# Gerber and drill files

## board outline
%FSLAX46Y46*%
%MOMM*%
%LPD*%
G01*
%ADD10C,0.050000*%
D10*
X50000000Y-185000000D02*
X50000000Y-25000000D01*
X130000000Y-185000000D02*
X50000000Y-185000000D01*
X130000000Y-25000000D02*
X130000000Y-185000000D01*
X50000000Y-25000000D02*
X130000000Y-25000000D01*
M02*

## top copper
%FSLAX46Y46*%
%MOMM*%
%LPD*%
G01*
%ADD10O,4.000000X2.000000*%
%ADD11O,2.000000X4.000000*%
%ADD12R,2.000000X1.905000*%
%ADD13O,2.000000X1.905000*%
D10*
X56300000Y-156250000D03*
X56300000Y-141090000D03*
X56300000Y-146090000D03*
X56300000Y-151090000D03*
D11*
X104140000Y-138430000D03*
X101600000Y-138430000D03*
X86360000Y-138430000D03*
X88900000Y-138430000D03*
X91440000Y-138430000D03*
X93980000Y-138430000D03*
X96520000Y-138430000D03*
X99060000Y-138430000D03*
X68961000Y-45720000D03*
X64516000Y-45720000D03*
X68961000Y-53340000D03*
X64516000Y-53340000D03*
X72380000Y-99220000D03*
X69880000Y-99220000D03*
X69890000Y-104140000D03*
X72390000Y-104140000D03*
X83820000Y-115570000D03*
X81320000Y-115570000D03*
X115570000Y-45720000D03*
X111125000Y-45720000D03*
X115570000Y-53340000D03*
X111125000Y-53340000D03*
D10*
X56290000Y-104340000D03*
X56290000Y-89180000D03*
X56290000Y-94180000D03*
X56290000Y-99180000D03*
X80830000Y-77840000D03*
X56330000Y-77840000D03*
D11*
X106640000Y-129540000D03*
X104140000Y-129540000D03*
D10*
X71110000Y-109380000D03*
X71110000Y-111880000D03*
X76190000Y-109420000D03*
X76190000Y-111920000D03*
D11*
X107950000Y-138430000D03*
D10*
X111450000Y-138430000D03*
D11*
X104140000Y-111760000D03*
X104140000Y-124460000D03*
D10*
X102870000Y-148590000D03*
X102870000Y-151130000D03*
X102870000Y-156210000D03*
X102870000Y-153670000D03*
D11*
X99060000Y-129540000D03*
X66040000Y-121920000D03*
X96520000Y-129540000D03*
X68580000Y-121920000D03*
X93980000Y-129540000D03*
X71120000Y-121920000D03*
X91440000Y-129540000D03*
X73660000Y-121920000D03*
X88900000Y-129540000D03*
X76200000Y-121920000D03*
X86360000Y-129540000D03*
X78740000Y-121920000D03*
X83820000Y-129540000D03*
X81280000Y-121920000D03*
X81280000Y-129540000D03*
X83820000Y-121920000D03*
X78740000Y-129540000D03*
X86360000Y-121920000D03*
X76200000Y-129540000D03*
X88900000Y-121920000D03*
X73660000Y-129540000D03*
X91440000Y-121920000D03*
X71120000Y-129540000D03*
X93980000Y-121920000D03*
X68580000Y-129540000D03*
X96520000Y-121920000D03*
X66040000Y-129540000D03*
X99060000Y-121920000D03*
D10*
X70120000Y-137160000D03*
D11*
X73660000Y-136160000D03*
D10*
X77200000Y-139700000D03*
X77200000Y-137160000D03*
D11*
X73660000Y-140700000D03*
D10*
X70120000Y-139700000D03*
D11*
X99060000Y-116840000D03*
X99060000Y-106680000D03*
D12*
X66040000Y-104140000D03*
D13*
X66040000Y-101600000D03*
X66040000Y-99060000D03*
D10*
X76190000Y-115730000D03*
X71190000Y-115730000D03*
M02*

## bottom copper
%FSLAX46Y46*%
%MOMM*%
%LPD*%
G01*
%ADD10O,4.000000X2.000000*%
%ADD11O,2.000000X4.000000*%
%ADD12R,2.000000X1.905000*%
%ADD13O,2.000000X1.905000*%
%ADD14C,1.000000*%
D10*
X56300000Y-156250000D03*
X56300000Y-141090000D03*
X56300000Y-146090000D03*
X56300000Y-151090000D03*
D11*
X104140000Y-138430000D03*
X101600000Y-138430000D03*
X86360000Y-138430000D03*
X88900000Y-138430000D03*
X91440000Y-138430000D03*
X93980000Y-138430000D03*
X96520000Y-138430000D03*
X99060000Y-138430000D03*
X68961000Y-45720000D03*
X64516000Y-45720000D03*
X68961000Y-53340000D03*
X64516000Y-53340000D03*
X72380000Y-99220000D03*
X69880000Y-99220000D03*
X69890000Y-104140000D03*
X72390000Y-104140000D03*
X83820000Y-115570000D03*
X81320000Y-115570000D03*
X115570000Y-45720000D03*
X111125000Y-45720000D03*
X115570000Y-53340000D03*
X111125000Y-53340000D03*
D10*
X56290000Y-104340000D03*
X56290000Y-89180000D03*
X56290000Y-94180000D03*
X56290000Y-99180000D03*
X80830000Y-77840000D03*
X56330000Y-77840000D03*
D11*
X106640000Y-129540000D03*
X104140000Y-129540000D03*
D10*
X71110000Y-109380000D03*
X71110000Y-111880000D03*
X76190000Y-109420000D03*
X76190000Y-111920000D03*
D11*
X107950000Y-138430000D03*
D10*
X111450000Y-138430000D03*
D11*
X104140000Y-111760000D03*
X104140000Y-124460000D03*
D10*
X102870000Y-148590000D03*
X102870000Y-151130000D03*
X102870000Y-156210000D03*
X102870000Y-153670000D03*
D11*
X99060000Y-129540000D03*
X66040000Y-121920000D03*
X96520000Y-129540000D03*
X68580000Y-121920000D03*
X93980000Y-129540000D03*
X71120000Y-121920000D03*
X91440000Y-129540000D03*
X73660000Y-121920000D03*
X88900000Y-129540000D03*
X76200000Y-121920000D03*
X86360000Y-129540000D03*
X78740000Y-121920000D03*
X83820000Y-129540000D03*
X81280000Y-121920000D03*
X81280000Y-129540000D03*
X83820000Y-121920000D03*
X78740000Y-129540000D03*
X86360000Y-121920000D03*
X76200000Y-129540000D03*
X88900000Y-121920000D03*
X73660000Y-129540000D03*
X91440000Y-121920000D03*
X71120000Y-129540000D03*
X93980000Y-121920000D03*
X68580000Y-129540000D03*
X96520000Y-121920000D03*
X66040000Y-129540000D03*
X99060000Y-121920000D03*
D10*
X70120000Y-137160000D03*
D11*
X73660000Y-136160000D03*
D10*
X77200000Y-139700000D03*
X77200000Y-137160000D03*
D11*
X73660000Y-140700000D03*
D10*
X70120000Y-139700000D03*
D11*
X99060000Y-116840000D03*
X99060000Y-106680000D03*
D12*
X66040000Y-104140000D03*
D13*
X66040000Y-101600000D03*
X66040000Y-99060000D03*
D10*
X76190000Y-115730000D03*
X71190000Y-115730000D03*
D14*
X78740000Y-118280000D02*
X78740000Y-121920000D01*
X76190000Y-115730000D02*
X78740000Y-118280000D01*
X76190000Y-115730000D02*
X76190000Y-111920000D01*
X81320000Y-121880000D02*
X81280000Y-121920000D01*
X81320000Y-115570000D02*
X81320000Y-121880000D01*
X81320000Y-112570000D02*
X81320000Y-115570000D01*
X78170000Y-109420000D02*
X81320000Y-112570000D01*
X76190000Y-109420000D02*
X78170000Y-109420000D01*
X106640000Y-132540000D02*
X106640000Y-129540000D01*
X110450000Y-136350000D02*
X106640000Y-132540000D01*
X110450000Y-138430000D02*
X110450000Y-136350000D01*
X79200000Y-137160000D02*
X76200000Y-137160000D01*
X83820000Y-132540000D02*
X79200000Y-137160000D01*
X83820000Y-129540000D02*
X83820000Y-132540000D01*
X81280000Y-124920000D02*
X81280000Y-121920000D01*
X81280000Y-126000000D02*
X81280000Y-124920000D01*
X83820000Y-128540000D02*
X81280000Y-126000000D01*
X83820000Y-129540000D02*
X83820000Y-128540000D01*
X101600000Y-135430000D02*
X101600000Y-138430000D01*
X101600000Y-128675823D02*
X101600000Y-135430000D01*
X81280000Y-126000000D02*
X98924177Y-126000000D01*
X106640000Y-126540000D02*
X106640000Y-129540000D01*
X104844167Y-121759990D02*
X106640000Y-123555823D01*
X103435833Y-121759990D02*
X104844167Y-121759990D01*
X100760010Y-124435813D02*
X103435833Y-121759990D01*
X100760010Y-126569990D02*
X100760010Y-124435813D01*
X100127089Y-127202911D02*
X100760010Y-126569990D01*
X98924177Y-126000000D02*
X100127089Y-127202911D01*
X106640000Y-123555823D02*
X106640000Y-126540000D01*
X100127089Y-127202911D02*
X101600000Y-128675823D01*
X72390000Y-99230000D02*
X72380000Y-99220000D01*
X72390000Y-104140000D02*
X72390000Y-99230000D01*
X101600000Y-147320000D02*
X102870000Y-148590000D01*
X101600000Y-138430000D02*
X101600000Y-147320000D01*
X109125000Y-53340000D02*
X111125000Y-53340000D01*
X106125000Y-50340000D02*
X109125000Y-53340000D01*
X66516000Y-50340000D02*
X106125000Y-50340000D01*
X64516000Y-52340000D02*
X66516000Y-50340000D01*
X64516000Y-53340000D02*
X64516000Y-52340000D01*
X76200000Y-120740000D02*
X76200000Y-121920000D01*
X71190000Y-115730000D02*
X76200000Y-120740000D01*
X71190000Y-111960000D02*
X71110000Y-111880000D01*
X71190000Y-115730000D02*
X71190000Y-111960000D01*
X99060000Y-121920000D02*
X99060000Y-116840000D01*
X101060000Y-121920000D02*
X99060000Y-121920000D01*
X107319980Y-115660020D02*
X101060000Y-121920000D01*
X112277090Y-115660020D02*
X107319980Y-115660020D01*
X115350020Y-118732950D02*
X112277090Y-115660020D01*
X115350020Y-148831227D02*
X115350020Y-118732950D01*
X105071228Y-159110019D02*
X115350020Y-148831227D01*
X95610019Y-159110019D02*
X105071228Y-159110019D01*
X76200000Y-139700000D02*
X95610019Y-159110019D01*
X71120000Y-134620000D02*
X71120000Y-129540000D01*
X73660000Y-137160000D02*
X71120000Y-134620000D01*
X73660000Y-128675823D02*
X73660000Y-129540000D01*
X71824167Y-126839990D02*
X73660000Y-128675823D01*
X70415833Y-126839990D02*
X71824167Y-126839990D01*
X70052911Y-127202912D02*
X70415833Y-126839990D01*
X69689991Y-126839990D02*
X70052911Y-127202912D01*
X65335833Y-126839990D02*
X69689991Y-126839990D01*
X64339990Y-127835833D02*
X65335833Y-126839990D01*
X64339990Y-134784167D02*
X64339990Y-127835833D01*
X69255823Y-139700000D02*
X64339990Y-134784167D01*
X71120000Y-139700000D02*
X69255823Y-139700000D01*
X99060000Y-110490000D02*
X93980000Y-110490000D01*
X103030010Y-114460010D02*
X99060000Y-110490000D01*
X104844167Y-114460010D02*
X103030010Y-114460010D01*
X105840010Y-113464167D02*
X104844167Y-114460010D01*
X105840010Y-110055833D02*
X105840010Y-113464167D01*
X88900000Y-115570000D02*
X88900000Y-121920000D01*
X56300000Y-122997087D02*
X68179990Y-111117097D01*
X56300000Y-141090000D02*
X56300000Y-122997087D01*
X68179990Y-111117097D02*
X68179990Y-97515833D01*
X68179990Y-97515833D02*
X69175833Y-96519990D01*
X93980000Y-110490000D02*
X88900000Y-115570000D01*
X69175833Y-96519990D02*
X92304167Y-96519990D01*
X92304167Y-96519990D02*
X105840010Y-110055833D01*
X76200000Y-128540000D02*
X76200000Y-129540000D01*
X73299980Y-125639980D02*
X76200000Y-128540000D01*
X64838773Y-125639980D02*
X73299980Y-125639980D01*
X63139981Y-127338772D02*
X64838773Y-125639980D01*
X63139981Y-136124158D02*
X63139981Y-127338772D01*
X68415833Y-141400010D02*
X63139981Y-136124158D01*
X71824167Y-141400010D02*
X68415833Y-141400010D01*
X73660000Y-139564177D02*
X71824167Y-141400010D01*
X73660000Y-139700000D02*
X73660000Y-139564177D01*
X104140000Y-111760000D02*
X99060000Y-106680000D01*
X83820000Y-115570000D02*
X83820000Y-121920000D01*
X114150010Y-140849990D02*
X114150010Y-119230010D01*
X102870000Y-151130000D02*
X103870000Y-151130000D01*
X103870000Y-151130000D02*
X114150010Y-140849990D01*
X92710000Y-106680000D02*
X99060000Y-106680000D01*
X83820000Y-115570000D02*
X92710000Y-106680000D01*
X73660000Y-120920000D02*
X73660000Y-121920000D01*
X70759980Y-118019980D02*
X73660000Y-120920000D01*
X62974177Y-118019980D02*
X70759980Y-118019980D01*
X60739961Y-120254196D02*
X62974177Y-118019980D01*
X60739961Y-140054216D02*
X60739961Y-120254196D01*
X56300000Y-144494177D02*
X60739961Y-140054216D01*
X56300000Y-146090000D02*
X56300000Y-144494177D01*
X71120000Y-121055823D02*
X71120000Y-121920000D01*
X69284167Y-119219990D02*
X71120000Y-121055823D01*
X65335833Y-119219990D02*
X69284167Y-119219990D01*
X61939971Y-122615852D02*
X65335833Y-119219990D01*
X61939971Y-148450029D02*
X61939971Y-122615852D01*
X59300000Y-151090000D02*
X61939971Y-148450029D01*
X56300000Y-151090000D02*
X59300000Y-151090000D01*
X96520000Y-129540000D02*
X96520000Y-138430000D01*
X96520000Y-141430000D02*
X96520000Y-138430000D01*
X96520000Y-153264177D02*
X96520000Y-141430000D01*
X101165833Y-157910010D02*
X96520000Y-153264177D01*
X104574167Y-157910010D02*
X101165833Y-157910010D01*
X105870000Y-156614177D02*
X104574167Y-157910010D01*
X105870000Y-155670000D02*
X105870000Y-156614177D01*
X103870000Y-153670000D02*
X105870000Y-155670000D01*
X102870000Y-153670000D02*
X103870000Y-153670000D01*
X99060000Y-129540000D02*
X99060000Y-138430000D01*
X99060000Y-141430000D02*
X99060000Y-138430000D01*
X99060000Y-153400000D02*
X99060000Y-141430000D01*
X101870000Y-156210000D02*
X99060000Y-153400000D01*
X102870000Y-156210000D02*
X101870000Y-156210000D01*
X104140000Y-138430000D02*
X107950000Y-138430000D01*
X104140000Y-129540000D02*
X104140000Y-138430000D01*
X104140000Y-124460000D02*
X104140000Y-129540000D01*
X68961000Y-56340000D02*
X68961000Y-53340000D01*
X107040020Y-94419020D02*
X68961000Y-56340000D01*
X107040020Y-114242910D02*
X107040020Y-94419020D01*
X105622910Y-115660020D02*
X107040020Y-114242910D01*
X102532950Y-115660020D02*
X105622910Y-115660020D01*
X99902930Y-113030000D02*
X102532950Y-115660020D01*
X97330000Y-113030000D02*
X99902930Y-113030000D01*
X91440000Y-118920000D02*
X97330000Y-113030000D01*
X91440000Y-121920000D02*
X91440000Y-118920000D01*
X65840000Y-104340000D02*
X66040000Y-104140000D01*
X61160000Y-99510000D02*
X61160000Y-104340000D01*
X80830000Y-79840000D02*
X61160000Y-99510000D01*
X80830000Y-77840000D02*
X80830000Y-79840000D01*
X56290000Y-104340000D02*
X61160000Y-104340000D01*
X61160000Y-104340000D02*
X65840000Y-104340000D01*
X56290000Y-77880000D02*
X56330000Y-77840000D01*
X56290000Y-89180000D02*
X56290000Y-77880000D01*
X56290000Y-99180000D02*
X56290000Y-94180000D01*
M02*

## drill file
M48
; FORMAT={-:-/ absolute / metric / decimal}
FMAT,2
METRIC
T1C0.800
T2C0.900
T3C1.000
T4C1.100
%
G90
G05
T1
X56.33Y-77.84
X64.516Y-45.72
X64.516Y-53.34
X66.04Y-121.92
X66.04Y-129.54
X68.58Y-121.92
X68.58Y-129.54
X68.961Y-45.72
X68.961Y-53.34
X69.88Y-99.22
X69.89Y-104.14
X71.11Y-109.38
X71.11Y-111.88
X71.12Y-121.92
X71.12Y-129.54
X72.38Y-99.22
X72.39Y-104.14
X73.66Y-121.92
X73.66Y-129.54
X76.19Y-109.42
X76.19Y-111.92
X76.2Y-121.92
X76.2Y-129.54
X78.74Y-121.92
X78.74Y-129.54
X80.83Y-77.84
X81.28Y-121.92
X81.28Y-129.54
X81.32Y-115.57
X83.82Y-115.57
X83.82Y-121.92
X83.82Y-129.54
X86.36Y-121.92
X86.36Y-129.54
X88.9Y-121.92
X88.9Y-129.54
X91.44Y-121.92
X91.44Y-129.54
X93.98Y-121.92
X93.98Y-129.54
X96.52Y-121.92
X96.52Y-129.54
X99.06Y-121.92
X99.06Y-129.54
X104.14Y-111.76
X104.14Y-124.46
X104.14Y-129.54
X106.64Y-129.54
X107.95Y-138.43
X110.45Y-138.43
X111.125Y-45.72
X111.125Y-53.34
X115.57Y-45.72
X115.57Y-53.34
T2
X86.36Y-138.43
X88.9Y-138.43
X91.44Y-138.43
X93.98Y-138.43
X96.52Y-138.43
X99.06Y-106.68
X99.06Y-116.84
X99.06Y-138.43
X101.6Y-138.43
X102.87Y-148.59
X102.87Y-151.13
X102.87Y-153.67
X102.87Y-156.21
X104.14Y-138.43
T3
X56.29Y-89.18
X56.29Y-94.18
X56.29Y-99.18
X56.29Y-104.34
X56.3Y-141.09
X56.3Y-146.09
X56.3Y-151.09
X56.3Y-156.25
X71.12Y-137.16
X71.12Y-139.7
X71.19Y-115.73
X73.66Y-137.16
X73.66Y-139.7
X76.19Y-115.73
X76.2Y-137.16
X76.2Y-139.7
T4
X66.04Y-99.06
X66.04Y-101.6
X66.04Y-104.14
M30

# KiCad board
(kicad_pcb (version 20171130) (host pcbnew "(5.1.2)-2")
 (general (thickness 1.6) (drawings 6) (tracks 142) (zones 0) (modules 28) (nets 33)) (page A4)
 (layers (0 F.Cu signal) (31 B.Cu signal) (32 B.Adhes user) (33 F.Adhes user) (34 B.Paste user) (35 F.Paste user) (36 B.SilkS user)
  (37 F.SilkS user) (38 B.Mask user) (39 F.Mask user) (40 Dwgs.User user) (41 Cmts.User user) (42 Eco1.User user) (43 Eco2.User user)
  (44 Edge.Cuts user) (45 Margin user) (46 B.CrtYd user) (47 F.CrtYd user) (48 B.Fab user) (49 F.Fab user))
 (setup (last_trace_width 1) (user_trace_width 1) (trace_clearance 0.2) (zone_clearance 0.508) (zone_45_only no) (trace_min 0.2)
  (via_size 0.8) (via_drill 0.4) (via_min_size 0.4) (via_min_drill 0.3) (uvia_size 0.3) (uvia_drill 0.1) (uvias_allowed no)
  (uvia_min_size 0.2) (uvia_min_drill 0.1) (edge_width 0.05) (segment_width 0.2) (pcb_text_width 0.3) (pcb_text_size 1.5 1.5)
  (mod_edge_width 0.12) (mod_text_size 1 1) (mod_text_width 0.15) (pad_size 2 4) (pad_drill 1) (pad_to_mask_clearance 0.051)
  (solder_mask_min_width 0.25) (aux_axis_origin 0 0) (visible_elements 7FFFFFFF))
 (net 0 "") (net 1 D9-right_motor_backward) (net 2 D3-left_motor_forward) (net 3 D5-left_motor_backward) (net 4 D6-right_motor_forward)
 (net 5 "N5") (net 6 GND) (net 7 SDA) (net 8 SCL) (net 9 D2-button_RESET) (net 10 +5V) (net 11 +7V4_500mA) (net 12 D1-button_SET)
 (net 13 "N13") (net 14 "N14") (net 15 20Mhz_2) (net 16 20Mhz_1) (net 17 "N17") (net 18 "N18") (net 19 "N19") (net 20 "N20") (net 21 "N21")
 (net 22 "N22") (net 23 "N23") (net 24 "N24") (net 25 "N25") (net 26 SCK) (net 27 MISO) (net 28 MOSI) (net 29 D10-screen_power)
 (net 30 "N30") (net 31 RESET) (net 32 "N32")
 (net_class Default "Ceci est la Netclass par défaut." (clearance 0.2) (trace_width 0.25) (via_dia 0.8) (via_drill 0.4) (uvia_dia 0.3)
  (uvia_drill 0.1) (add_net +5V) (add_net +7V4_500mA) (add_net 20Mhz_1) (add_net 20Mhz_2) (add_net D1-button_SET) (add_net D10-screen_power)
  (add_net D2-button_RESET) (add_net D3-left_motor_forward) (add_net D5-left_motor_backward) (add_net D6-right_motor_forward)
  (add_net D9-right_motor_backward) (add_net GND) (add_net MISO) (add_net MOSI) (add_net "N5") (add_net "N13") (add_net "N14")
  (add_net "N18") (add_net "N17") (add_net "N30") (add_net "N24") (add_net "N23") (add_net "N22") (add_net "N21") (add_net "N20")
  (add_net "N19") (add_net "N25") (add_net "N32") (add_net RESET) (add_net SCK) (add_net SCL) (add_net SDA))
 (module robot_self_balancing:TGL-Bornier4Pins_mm (layer F.Cu) (at 50.8 148.59 90)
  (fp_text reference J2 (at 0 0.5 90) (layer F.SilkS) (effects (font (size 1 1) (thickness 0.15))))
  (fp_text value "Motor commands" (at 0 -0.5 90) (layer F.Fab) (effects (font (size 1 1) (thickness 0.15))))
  (pad 5 thru_hole oval (at -7.66 5.5 90) (size 2 4) (drill 1) (layers *.Cu *.Mask) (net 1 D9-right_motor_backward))
  (pad 8 thru_hole oval (at 7.5 5.5 270) (size 2 4) (drill 1) (layers *.Cu *.Mask) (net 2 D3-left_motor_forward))
  (pad 7 thru_hole oval (at 2.5 5.5 90) (size 2 4) (drill 1) (layers *.Cu *.Mask) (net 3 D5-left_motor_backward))
  (pad 6 thru_hole oval (at -2.5 5.5 90) (size 2 4) (drill 1) (layers *.Cu *.Mask) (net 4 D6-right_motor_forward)))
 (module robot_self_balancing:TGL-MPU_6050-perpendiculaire (layer F.Cu) (at 95.25 142.24 180)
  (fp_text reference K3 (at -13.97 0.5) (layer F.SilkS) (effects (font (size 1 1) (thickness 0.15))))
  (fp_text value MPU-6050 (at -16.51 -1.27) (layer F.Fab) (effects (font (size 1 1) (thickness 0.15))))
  (pad 13 thru_hole oval (at -8.89 3.81 180) (size 2 4) (drill 0.9) (layers *.Cu *.Mask) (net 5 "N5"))
  (pad 18 thru_hole oval (at -6.35 3.81 180) (size 2 4) (drill 0.9) (layers *.Cu *.Mask) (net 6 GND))
  (pad "" thru_hole oval (at 8.89 3.81 180) (size 2 4) (drill 0.9) (layers *.Cu *.Mask))
  (pad "" thru_hole oval (at 6.35 3.81 180) (size 2 4) (drill 0.9) (layers *.Cu *.Mask))
  (pad "" thru_hole oval (at 3.81 3.81 180) (size 2 4) (drill 0.9) (layers *.Cu *.Mask))
  (pad "" thru_hole oval (at 1.27 3.81 180) (size 2 4) (drill 0.9) (layers *.Cu *.Mask))
  (pad 24 thru_hole oval (at -1.27 3.81 180) (size 2 4) (drill 0.9) (layers *.Cu *.Mask) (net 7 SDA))
  (pad 23 thru_hole oval (at -3.81 3.81 180) (size 2 4) (drill 0.9) (layers *.Cu *.Mask) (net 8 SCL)))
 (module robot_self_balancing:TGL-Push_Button (layer F.Cu) (at 62.23 49.53 90)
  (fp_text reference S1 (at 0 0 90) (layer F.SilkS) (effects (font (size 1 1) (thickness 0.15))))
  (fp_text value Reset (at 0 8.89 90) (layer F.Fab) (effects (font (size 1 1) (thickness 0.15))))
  (pad 4 thru_hole oval (at 3.81 6.731 90) (size 4 2) (drill 0.8) (layers *.Cu *.Mask))
  (pad 3 thru_hole oval (at 3.81 2.286 90) (size 4 2) (drill 0.8) (layers *.Cu *.Mask))
  (pad 2 thru_hole oval (at -3.81 6.731 90) (size 4 2) (drill 0.8) (layers *.Cu *.Mask) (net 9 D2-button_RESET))
  (pad 1 thru_hole oval (at -3.81 2.286 90) (size 4 2) (drill 0.8) (layers *.Cu *.Mask) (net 6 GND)))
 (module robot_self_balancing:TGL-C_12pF (layer F.Cu) (at 69.88 99.22)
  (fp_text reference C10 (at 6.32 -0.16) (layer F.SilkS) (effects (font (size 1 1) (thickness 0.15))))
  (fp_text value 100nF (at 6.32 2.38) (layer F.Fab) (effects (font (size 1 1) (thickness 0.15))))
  (pad 2 thru_hole oval (at 2.5 0) (size 2 4) (drill 0.8) (layers *.Cu *.Mask) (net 6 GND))
  (pad 1 thru_hole oval (at 0 0) (size 2 4) (drill 0.8) (layers *.Cu *.Mask) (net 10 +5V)))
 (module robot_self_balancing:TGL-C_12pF (layer F.Cu) (at 72.39 104.14 180)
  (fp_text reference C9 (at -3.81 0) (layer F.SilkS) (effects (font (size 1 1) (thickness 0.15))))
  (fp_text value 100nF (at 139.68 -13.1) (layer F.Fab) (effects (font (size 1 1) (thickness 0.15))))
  (pad 2 thru_hole oval (at 2.5 0 180) (size 2 4) (drill 0.8) (layers *.Cu *.Mask) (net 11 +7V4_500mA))
  (pad 1 thru_hole oval (at 0 0 180) (size 2 4) (drill 0.8) (layers *.Cu *.Mask) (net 6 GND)))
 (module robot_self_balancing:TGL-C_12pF (layer F.Cu) (at 81.32 115.57)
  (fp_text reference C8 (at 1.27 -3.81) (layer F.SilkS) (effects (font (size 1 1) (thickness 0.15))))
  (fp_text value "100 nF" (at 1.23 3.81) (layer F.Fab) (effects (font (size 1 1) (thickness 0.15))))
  (pad 2 thru_hole oval (at 2.5 0) (size 2 4) (drill 0.8) (layers *.Cu *.Mask) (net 10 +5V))
  (pad 1 thru_hole oval (at 0 0) (size 2 4) (drill 0.8) (layers *.Cu *.Mask) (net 6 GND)))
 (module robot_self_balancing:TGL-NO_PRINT (layer F.Cu) (at -48.26 104.14)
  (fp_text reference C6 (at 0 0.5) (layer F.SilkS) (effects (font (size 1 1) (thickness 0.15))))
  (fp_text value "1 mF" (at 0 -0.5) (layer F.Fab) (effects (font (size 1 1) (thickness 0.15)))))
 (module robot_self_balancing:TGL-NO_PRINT (layer F.Cu) (at -58.42 102.87)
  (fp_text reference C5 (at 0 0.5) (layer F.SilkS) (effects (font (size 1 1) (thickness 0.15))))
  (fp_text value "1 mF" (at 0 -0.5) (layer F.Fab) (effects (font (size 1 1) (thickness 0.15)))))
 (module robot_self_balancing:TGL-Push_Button (layer F.Cu) (at 108.839 49.53 90)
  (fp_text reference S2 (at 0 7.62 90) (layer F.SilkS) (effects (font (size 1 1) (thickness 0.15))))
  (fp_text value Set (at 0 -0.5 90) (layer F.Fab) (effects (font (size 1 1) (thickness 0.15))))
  (pad 4 thru_hole oval (at 3.81 6.731 90) (size 4 2) (drill 0.8) (layers *.Cu *.Mask))
  (pad 3 thru_hole oval (at 3.81 2.286 90) (size 4 2) (drill 0.8) (layers *.Cu *.Mask))
  (pad 2 thru_hole oval (at -3.81 6.731 90) (size 4 2) (drill 0.8) (layers *.Cu *.Mask) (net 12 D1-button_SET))
  (pad 1 thru_hole oval (at -3.81 2.286 90) (size 4 2) (drill 0.8) (layers *.Cu *.Mask) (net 6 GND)))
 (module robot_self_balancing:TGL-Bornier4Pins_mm (layer F.Cu) (at 50.79 96.68 90)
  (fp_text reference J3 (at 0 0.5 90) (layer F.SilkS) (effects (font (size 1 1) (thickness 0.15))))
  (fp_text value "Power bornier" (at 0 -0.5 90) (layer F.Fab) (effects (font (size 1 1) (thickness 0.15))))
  (pad 8 thru_hole oval (at -7.66 5.5 90) (size 2 4) (drill 1) (layers *.Cu *.Mask) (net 11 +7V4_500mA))
  (pad 5 thru_hole oval (at 7.5 5.5 270) (size 2 4) (drill 1) (layers *.Cu *.Mask) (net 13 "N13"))
  (pad 7 thru_hole oval (at 2.5 5.5 90) (size 2 4) (drill 1) (layers *.Cu *.Mask) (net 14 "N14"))
  (pad 6 thru_hole oval (at -2.5 5.5 90) (size 2 4) (drill 1) (layers *.Cu *.Mask) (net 14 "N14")))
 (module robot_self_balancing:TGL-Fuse (layer F.Cu) (at 68.58 85.09 180)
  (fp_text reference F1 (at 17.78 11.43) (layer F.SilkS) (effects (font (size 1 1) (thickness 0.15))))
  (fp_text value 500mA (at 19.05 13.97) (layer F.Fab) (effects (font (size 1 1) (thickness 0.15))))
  (pad 1 thru_hole oval (at -12.25 7.25 270) (size 2 4) (drill 0.8) (layers *.Cu *.Mask) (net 11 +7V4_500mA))
  (pad 2 thru_hole oval (at 12.25 7.25 270) (size 2 4) (drill 0.8) (layers *.Cu *.Mask) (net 13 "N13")))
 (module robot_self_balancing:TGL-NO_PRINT (layer F.Cu) (at -48.26 87.63)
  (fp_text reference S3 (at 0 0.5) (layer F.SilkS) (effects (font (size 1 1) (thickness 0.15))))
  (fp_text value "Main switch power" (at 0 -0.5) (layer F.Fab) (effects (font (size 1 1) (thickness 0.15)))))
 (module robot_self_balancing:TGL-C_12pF (layer F.Cu) (at 104.14 129.54)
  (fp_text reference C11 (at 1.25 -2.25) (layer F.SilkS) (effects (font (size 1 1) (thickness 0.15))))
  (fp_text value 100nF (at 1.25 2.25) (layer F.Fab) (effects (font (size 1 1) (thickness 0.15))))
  (pad 2 thru_hole oval (at 2.5 0) (size 2 4) (drill 0.8) (layers *.Cu *.Mask) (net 6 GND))
  (pad 1 thru_hole oval (at 0 0) (size 2 4) (drill 0.8) (layers *.Cu *.Mask) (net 5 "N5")))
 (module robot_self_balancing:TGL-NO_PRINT (layer F.Cu) (at -48.26 74.93)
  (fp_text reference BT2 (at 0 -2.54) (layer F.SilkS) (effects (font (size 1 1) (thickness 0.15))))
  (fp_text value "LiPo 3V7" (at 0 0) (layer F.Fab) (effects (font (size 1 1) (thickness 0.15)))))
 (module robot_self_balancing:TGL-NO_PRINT (layer F.Cu) (at -48.26 62.23)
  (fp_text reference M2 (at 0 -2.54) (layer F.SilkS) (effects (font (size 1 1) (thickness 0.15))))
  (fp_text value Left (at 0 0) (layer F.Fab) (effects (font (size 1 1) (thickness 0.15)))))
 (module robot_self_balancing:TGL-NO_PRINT (layer F.Cu) (at -48.26 50.8)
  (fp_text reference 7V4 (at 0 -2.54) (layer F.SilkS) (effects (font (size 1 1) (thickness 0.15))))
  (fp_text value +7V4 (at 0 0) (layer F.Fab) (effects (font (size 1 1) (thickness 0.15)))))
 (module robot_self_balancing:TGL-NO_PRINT (layer F.Cu) (at -48.26 38.1)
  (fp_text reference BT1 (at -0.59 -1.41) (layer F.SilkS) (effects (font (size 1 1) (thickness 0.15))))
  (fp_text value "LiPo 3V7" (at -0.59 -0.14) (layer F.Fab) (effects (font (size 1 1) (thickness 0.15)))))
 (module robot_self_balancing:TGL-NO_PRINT (layer F.Cu) (at -48.26 27.94)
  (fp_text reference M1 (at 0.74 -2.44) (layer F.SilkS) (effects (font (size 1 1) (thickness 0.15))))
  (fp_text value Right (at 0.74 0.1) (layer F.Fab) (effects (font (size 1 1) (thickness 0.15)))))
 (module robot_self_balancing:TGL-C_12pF (layer F.Cu) (at 71.11 111.88 90)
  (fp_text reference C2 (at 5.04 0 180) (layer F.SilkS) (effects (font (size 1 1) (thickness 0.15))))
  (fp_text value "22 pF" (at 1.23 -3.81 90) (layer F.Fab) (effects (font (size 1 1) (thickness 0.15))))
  (pad 2 thru_hole oval (at 2.5 0 90) (size 2 4) (drill 0.8) (layers *.Cu *.Mask) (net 6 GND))
  (pad 1 thru_hole oval (at 0 0 90) (size 2 4) (drill 0.8) (layers *.Cu *.Mask) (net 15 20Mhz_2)))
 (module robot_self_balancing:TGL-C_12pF (layer F.Cu) (at 76.19 111.92 90)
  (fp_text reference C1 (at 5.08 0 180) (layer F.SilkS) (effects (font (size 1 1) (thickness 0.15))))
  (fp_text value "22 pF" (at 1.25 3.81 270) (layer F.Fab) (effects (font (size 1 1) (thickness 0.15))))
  (pad 2 thru_hole oval (at 2.5 0 90) (size 2 4) (drill 0.8) (layers *.Cu *.Mask) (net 6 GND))
  (pad 1 thru_hole oval (at 0 0 90) (size 2 4) (drill 0.8) (layers *.Cu *.Mask) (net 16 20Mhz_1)))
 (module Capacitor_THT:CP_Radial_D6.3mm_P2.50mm (layer F.Cu) (at 107.95 138.43)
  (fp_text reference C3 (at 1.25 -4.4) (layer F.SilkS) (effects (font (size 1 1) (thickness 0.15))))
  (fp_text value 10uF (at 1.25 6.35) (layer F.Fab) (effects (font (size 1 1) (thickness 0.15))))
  (pad 1 thru_hole oval (at 0 0) (size 2 4) (drill 0.8) (layers *.Cu *.Mask) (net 5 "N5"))
  (pad 2 thru_hole oval (at 2.5 0) (size 4 2) (drill 0.8 (offset 1 0)) (layers *.Cu *.Mask) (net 6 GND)))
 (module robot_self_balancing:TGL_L (layer F.Cu) (at 104.14 124.46 90)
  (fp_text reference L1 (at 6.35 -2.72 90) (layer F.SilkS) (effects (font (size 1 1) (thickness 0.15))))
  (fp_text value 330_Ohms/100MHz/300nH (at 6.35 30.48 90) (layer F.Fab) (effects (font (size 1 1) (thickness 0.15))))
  (pad 2 thru_hole oval (at 12.7 0 90) (size 4 2) (drill 0.8) (layers *.Cu *.Mask) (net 10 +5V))
  (pad 1 thru_hole oval (at 0 0 90) (size 4 2) (drill 0.8) (layers *.Cu *.Mask) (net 5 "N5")))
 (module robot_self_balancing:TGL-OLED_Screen (layer F.Cu) (at 106.68 152.4 270)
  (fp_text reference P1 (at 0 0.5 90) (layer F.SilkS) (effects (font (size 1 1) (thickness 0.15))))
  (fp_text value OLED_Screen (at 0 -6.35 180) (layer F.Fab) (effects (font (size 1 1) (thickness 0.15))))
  (pad 1 thru_hole oval (at -3.81 3.81 270) (size 2 4) (drill 0.9) (layers *.Cu *.Mask) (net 6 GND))
  (pad 2 thru_hole oval (at -1.27 3.81 270) (size 2 4) (drill 0.9) (layers *.Cu *.Mask) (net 10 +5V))
  (pad 4 thru_hole oval (at 3.81 3.81 270) (size 2 4) (drill 0.9) (layers *.Cu *.Mask) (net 8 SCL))
  (pad 3 thru_hole oval (at 1.27 3.81 270) (size 2 4) (drill 0.9) (layers *.Cu *.Mask) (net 7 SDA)))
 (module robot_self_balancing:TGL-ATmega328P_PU (layer F.Cu) (at 99.06 121.92 270)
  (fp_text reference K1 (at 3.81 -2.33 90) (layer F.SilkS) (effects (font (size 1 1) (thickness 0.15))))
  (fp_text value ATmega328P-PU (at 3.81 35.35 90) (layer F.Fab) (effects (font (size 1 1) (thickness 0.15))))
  (pad 28 thru_hole oval (at 7.62 0 270) (size 4 2) (drill 0.8) (layers *.Cu *.Mask) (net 8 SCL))
  (pad 14 thru_hole oval (at 0 33.02 270) (size 4 2) (drill 0.8) (layers *.Cu *.Mask) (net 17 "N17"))
  (pad 27 thru_hole oval (at 7.62 2.54 270) (size 4 2) (drill 0.8) (layers *.Cu *.Mask) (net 7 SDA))
  (pad 13 thru_hole oval (at 0 30.48 270) (size 4 2) (drill 0.8) (layers *.Cu *.Mask) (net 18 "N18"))
  (pad 26 thru_hole oval (at 7.62 5.08 270) (size 4 2) (drill 0.8) (layers *.Cu *.Mask) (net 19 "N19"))
  (pad 12 thru_hole oval (at 0 27.94 270) (size 4 2) (drill 0.8) (layers *.Cu *.Mask) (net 4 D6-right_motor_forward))
  (pad 25 thru_hole oval (at 7.62 7.62 270) (size 4 2) (drill 0.8) (layers *.Cu *.Mask) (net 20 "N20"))
  (pad 11 thru_hole oval (at 0 25.4 270) (size 4 2) (drill 0.8) (layers *.Cu *.Mask) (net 3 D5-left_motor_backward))
  (pad 24 thru_hole oval (at 7.62 10.16 270) (size 4 2) (drill 0.8) (layers *.Cu *.Mask) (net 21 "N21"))
  (pad 10 thru_hole oval (at 0 22.86 270) (size 4 2) (drill 0.8) (layers *.Cu *.Mask) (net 15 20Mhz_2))
  (pad 23 thru_hole oval (at 7.62 12.7 270) (size 4 2) (drill 0.8) (layers *.Cu *.Mask) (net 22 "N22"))
  (pad 9 thru_hole oval (at 0 20.32 270) (size 4 2) (drill 0.8) (layers *.Cu *.Mask) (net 16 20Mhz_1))
  (pad 22 thru_hole oval (at 7.62 15.24 270) (size 4 2) (drill 0.8) (layers *.Cu *.Mask) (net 6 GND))
  (pad 8 thru_hole oval (at 0 17.78 270) (size 4 2) (drill 0.8) (layers *.Cu *.Mask) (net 6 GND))
  (pad 21 thru_hole oval (at 7.62 17.78 270) (size 4 2) (drill 0.8) (layers *.Cu *.Mask) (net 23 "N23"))
  (pad 7 thru_hole oval (at 0 15.24 270) (size 4 2) (drill 0.8) (layers *.Cu *.Mask) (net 10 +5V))
  (pad 20 thru_hole oval (at 7.62 20.32 270) (size 4 2) (drill 0.8) (layers *.Cu *.Mask) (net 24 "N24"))
  (pad 6 thru_hole oval (at 0 12.7 270) (size 4 2) (drill 0.8) (layers *.Cu *.Mask) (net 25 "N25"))
  (pad 19 thru_hole oval (at 7.62 22.86 270) (size 4 2) (drill 0.8) (layers *.Cu *.Mask) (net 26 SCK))
  (pad 5 thru_hole oval (at 0 10.16 270) (size 4 2) (drill 0.8) (layers *.Cu *.Mask) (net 2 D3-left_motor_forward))
  (pad 18 thru_hole oval (at 7.62 25.4 270) (size 4 2) (drill 0.8) (layers *.Cu *.Mask) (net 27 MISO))
  (pad 4 thru_hole oval (at 0 7.62 270) (size 4 2) (drill 0.8) (layers *.Cu *.Mask) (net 9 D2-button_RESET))
  (pad 17 thru_hole oval (at 7.62 27.94 270) (size 4 2) (drill 0.8) (layers *.Cu *.Mask) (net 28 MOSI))
  (pad 3 thru_hole oval (at 0 5.08 270) (size 4 2) (drill 0.8) (layers *.Cu *.Mask) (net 12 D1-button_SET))
  (pad 16 thru_hole oval (at 7.62 30.48 270) (size 4 2) (drill 0.8) (layers *.Cu *.Mask) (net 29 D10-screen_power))
  (pad 2 thru_hole oval (at 0 2.54 270) (size 4 2) (drill 0.8) (layers *.Cu *.Mask) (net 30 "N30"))
  (pad 15 thru_hole oval (at 7.62 33.02 270) (size 4 2) (drill 0.8) (layers *.Cu *.Mask) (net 1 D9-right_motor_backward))
  (pad 1 thru_hole oval (at 0 0 270) (size 4 2) (drill 0.8) (layers *.Cu *.Mask) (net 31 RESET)))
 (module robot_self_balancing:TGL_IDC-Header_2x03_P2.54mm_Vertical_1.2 (layer F.Cu) (at 71.12 139.7 90)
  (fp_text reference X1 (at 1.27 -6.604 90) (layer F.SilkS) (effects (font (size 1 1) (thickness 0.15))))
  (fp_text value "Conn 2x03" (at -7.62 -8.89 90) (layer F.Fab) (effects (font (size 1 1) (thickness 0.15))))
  (pad 2 thru_hole oval (at 2.54 0 90) (size 2 4) (drill 1 (offset 0 -1)) (layers *.Cu *.Mask) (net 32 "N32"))
  (pad 4 thru_hole oval (at 2.54 2.54 90) (size 4 2) (drill 1 (offset 1 0)) (layers *.Cu *.Mask) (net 28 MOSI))
  (pad 5 thru_hole oval (at 0 5.08 90) (size 2 4) (drill 1 (offset 0 1)) (layers *.Cu *.Mask) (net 31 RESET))
  (pad 6 thru_hole oval (at 2.54 5.08 90) (size 2 4) (drill 1 (offset 0 1)) (layers *.Cu *.Mask) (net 6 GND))
  (pad 3 thru_hole oval (at 0 2.54 90) (size 4 2) (drill 1 (offset -1 0)) (layers *.Cu *.Mask) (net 26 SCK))
  (pad 1 thru_hole oval (at 0 0 90) (size 2 4) (drill 1 (offset 0 -1)) (layers *.Cu *.Mask) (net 27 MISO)))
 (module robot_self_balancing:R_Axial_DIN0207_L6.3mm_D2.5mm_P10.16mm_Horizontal (layer F.Cu) (at 99.06 106.68 270)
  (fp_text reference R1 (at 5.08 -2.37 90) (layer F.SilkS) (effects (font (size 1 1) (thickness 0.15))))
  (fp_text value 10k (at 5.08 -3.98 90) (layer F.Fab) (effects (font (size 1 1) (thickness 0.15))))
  (pad 2 thru_hole oval (at 10.16 0 270) (size 4 2) (drill 0.9) (layers *.Cu *.Mask) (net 31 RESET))
  (pad 1 thru_hole oval (at 0 0 270) (size 4 2) (drill 0.9) (layers *.Cu *.Mask) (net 10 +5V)))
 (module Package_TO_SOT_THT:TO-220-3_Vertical (layer F.Cu) (at 66.04 104.14 90)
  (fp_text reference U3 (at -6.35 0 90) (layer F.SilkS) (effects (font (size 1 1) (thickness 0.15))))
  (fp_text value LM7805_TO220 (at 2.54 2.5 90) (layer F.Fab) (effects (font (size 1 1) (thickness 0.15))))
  (pad 1 thru_hole rect (at 0 0 90) (size 1.905 2) (drill 1.1) (layers *.Cu *.Mask) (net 11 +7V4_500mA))
  (pad 2 thru_hole oval (at 2.54 0 90) (size 1.905 2) (drill 1.1) (layers *.Cu *.Mask) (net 6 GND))
  (pad 3 thru_hole oval (at 5.08 0 90) (size 1.905 2) (drill 1.1) (layers *.Cu *.Mask) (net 10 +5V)))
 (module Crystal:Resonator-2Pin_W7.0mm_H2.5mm (layer F.Cu) (at 76.19 115.73 180)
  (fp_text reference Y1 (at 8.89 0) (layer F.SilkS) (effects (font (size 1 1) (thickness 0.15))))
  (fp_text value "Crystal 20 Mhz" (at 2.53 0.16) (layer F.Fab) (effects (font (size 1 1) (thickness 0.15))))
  (pad 1 thru_hole oval (at 0 0 180) (size 4 2) (drill 1) (layers *.Cu *.Mask) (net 16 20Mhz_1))
  (pad 2 thru_hole oval (at 5 0 180) (size 4 2) (drill 1) (layers *.Cu *.Mask) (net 15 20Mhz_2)))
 (gr_line (start 50 185) (end 50 25) (layer Edge.Cuts) (width 0.05))
 (gr_line (start 130 185) (end 50 185) (layer Edge.Cuts) (width 0.05))
 (gr_line (start 130 25) (end 130 185) (layer Edge.Cuts) (width 0.05))
 (gr_line (start 50 25) (end 130 25) (layer Edge.Cuts) (width 0.05))
 (segment (start 78.74 118.28) (end 78.74 121.92) (width 1) (layer B.Cu) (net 16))
 (segment (start 76.19 115.73) (end 78.74 118.28) (width 1) (layer B.Cu) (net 16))
 (segment (start 76.19 115.73) (end 76.19 111.92) (width 1) (layer B.Cu) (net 16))
 (segment (start 81.32 121.88) (end 81.28 121.92) (width 1) (layer B.Cu) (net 6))
 (segment (start 81.32 115.57) (end 81.32 121.88) (width 1) (layer B.Cu) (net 6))
 (segment (start 81.32 112.57) (end 81.32 115.57) (width 1) (layer B.Cu) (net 6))
 (segment (start 78.17 109.42) (end 81.32 112.57) (width 1) (layer B.Cu) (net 6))
 (segment (start 76.19 109.42) (end 78.17 109.42) (width 1) (layer B.Cu) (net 6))
 (segment (start 106.64 132.54) (end 106.64 129.54) (width 1) (layer B.Cu) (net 6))
 (segment (start 110.45 136.35) (end 106.64 132.54) (width 1) (layer B.Cu) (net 6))
 (segment (start 110.45 138.43) (end 110.45 136.35) (width 1) (layer B.Cu) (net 6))
 (segment (start 79.2 137.16) (end 76.2 137.16) (width 1) (layer B.Cu) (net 6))
 (segment (start 83.82 132.54) (end 79.2 137.16) (width 1) (layer B.Cu) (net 6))
 (segment (start 83.82 129.54) (end 83.82 132.54) (width 1) (layer B.Cu) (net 6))
 (segment (start 81.28 124.92) (end 81.28 121.92) (width 1) (layer B.Cu) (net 6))
 (segment (start 81.28 126) (end 81.28 124.92) (width 1) (layer B.Cu) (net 6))
 (segment (start 83.82 128.54) (end 81.28 126) (width 1) (layer B.Cu) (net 6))
 (segment (start 83.82 129.54) (end 83.82 128.54) (width 1) (layer B.Cu) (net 6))
 (segment (start 101.6 135.43) (end 101.6 138.43) (width 1) (layer B.Cu) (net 6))
 (segment (start 101.6 128.675823) (end 101.6 135.43) (width 1) (layer B.Cu) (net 6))
 (segment (start 81.28 126) (end 98.924177 126) (width 1) (layer B.Cu) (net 6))
 (segment (start 106.64 126.54) (end 106.64 129.54) (width 1) (layer B.Cu) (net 6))
 (segment (start 104.844167 121.75999) (end 106.64 123.555823) (width 1) (layer B.Cu) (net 6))
 (segment (start 103.435833 121.75999) (end 104.844167 121.75999) (width 1) (layer B.Cu) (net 6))
 (segment (start 100.76001 124.435813) (end 103.435833 121.75999) (width 1) (layer B.Cu) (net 6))
 (segment (start 100.76001 126.56999) (end 100.76001 124.435813) (width 1) (layer B.Cu) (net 6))
 (segment (start 100.127089 127.202911) (end 100.76001 126.56999) (width 1) (layer B.Cu) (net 6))
 (segment (start 98.924177 126) (end 100.127089 127.202911) (width 1) (layer B.Cu) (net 6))
 (segment (start 106.64 123.555823) (end 106.64 126.54) (width 1) (layer B.Cu) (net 6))
 (segment (start 100.127089 127.202911) (end 101.6 128.675823) (width 1) (layer B.Cu) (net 6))
 (segment (start 72.39 99.23) (end 72.38 99.22) (width 1) (layer B.Cu) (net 6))
 (segment (start 72.39 104.14) (end 72.39 99.23) (width 1) (layer B.Cu) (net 6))
 (segment (start 101.6 147.32) (end 102.87 148.59) (width 1) (layer B.Cu) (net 6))
 (segment (start 101.6 138.43) (end 101.6 147.32) (width 1) (layer B.Cu) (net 6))
 (segment (start 109.125 53.34) (end 111.125 53.34) (width 1) (layer B.Cu) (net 6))
 (segment (start 106.125 50.34) (end 109.125 53.34) (width 1) (layer B.Cu) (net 6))
 (segment (start 66.516 50.34) (end 106.125 50.34) (width 1) (layer B.Cu) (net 6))
 (segment (start 64.516 52.34) (end 66.516 50.34) (width 1) (layer B.Cu) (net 6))
 (segment (start 64.516 53.34) (end 64.516 52.34) (width 1) (layer B.Cu) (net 6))
 (segment (start 76.2 120.74) (end 76.2 121.92) (width 1) (layer B.Cu) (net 15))
 (segment (start 71.19 115.73) (end 76.2 120.74) (width 1) (layer B.Cu) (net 15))
 (segment (start 71.19 111.96) (end 71.11 111.88) (width 1) (layer B.Cu) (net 15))
 (segment (start 71.19 115.73) (end 71.19 111.96) (width 1) (layer B.Cu) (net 15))
 (segment (start 99.06 121.92) (end 99.06 116.84) (width 1) (layer B.Cu) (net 31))
 (segment (start 101.06 121.92) (end 99.06 121.92) (width 1) (layer B.Cu) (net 31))
 (segment (start 107.31998 115.66002) (end 101.06 121.92) (width 1) (layer B.Cu) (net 31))
 (segment (start 112.27709 115.66002) (end 107.31998 115.66002) (width 1) (layer B.Cu) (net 31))
 (segment (start 115.35002 118.73295) (end 112.27709 115.66002) (width 1) (layer B.Cu) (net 31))
 (segment (start 115.35002 148.831227) (end 115.35002 118.73295) (width 1) (layer B.Cu) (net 31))
 (segment (start 105.071228 159.110019) (end 115.35002 148.831227) (width 1) (layer B.Cu) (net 31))
 (segment (start 95.610019 159.110019) (end 105.071228 159.110019) (width 1) (layer B.Cu) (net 31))
 (segment (start 76.2 139.7) (end 95.610019 159.110019) (width 1) (layer B.Cu) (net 31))
 (segment (start 71.12 134.62) (end 71.12 129.54) (width 1) (layer B.Cu) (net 28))
 (segment (start 73.66 137.16) (end 71.12 134.62) (width 1) (layer B.Cu) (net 28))
 (segment (start 73.66 128.675823) (end 73.66 129.54) (width 1) (layer B.Cu) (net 27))
 (segment (start 71.824167 126.83999) (end 73.66 128.675823) (width 1) (layer B.Cu) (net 27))
 (segment (start 70.415833 126.83999) (end 71.824167 126.83999) (width 1) (layer B.Cu) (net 27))
 (segment (start 70.052911 127.202912) (end 70.415833 126.83999) (width 1) (layer B.Cu) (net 27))
 (segment (start 69.689991 126.83999) (end 70.052911 127.202912) (width 1) (layer B.Cu) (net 27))
 (segment (start 65.335833 126.83999) (end 69.689991 126.83999) (width 1) (layer B.Cu) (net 27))
 (segment (start 64.33999 127.835833) (end 65.335833 126.83999) (width 1) (layer B.Cu) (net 27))
 (segment (start 64.33999 134.784167) (end 64.33999 127.835833) (width 1) (layer B.Cu) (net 27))
 (segment (start 69.255823 139.7) (end 64.33999 134.784167) (width 1) (layer B.Cu) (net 27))
 (segment (start 71.12 139.7) (end 69.255823 139.7) (width 1) (layer B.Cu) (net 27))
 (segment (start 99.06 110.49) (end 93.98 110.49) (width 1) (layer B.Cu) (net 2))
 (segment (start 103.03001 114.46001) (end 99.06 110.49) (width 1) (layer B.Cu) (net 2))
 (segment (start 104.844167 114.46001) (end 103.03001 114.46001) (width 1) (layer B.Cu) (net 2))
 (segment (start 105.84001 113.464167) (end 104.844167 114.46001) (width 1) (layer B.Cu) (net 2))
 (segment (start 105.84001 110.055833) (end 105.84001 113.464167) (width 1) (layer B.Cu) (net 2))
 (segment (start 88.9 115.57) (end 88.9 121.92) (width 1) (layer B.Cu) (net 2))
 (segment (start 56.3 122.997087) (end 68.17999 111.117097) (width 1) (layer B.Cu) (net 2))
 (segment (start 56.3 141.09) (end 56.3 122.997087) (width 1) (layer B.Cu) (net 2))
 (segment (start 68.17999 111.117097) (end 68.17999 97.515833) (width 1) (layer B.Cu) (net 2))
 (segment (start 68.17999 97.515833) (end 69.175833 96.51999) (width 1) (layer B.Cu) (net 2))
 (segment (start 93.98 110.49) (end 88.9 115.57) (width 1) (layer B.Cu) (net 2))
 (segment (start 69.175833 96.51999) (end 92.304167 96.51999) (width 1) (layer B.Cu) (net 2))
 (segment (start 92.304167 96.51999) (end 105.84001 110.055833) (width 1) (layer B.Cu) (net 2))
 (segment (start 76.2 128.54) (end 76.2 129.54) (width 1) (layer B.Cu) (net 26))
 (segment (start 73.29998 125.63998) (end 76.2 128.54) (width 1) (layer B.Cu) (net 26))
 (segment (start 64.838773 125.63998) (end 73.29998 125.63998) (width 1) (layer B.Cu) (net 26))
 (segment (start 63.139981 127.338772) (end 64.838773 125.63998) (width 1) (layer B.Cu) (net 26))
 (segment (start 63.139981 136.124158) (end 63.139981 127.338772) (width 1) (layer B.Cu) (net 26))
 (segment (start 68.415833 141.40001) (end 63.139981 136.124158) (width 1) (layer B.Cu) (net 26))
 (segment (start 71.824167 141.40001) (end 68.415833 141.40001) (width 1) (layer B.Cu) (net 26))
 (segment (start 73.66 139.564177) (end 71.824167 141.40001) (width 1) (layer B.Cu) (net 26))
 (segment (start 73.66 139.7) (end 73.66 139.564177) (width 1) (layer B.Cu) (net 26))
 (segment (start 104.14 111.76) (end 99.06 106.68) (width 1) (layer B.Cu) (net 10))
 (segment (start 83.82 115.57) (end 83.82 121.92) (width 1) (layer B.Cu) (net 10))
 (segment (start 114.15001 140.84999) (end 114.15001 119.23001) (width 1) (layer B.Cu) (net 10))
 (segment (start 102.87 151.13) (end 103.87 151.13) (width 1) (layer B.Cu) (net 10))
 (segment (start 103.87 151.13) (end 114.15001 140.84999) (width 1) (layer B.Cu) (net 10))
 (segment (start 92.71 106.68) (end 99.06 106.68) (width 1) (layer B.Cu) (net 10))
 (segment (start 83.82 115.57) (end 92.71 106.68) (width 1) (layer B.Cu) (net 10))
 (segment (start 73.66 120.92) (end 73.66 121.92) (width 1) (layer B.Cu) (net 3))
 (segment (start 70.75998 118.01998) (end 73.66 120.92) (width 1) (layer B.Cu) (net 3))
 (segment (start 62.974177 118.01998) (end 70.75998 118.01998) (width 1) (layer B.Cu) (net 3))
 (segment (start 60.739961 120.254196) (end 62.974177 118.01998) (width 1) (layer B.Cu) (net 3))
 (segment (start 60.739961 140.054216) (end 60.739961 120.254196) (width 1) (layer B.Cu) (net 3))
 (segment (start 56.3 144.494177) (end 60.739961 140.054216) (width 1) (layer B.Cu) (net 3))
 (segment (start 56.3 146.09) (end 56.3 144.494177) (width 1) (layer B.Cu) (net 3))
 (segment (start 71.12 121.055823) (end 71.12 121.92) (width 1) (layer B.Cu) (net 4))
 (segment (start 69.284167 119.21999) (end 71.12 121.055823) (width 1) (layer B.Cu) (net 4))
 (segment (start 65.335833 119.21999) (end 69.284167 119.21999) (width 1) (layer B.Cu) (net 4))
 (segment (start 61.939971 122.615852) (end 65.335833 119.21999) (width 1) (layer B.Cu) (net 4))
 (segment (start 61.939971 148.450029) (end 61.939971 122.615852) (width 1) (layer B.Cu) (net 4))
 (segment (start 59.3 151.09) (end 61.939971 148.450029) (width 1) (layer B.Cu) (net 4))
 (segment (start 56.3 151.09) (end 59.3 151.09) (width 1) (layer B.Cu) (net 4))
 (segment (start 96.52 129.54) (end 96.52 138.43) (width 1) (layer B.Cu) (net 7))
 (segment (start 96.52 141.43) (end 96.52 138.43) (width 1) (layer B.Cu) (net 7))
 (segment (start 96.52 153.264177) (end 96.52 141.43) (width 1) (layer B.Cu) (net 7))
 (segment (start 101.165833 157.91001) (end 96.52 153.264177) (width 1) (layer B.Cu) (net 7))
 (segment (start 104.574167 157.91001) (end 101.165833 157.91001) (width 1) (layer B.Cu) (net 7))
 (segment (start 105.87 156.614177) (end 104.574167 157.91001) (width 1) (layer B.Cu) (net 7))
 (segment (start 105.87 155.67) (end 105.87 156.614177) (width 1) (layer B.Cu) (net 7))
 (segment (start 103.87 153.67) (end 105.87 155.67) (width 1) (layer B.Cu) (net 7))
 (segment (start 102.87 153.67) (end 103.87 153.67) (width 1) (layer B.Cu) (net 7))
 (segment (start 99.06 129.54) (end 99.06 138.43) (width 1) (layer B.Cu) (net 8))
 (segment (start 99.06 141.43) (end 99.06 138.43) (width 1) (layer B.Cu) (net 8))
 (segment (start 99.06 153.4) (end 99.06 141.43) (width 1) (layer B.Cu) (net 8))
 (segment (start 101.87 156.21) (end 99.06 153.4) (width 1) (layer B.Cu) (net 8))
 (segment (start 102.87 156.21) (end 101.87 156.21) (width 1) (layer B.Cu) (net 8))
 (segment (start 104.14 138.43) (end 107.95 138.43) (width 1) (layer B.Cu) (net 5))
 (segment (start 104.14 129.54) (end 104.14 138.43) (width 1) (layer B.Cu) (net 5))
 (segment (start 104.14 124.46) (end 104.14 129.54) (width 1) (layer B.Cu) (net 5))
 (segment (start 68.961 56.34) (end 68.961 53.34) (width 1) (layer B.Cu) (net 9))
 (segment (start 107.04002 94.41902) (end 68.961 56.34) (width 1) (layer B.Cu) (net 9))
 (segment (start 107.04002 114.24291) (end 107.04002 94.41902) (width 1) (layer B.Cu) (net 9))
 (segment (start 105.62291 115.66002) (end 107.04002 114.24291) (width 1) (layer B.Cu) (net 9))
 (segment (start 102.53295 115.66002) (end 105.62291 115.66002) (width 1) (layer B.Cu) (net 9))
 (segment (start 99.90293 113.03) (end 102.53295 115.66002) (width 1) (layer B.Cu) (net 9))
 (segment (start 97.33 113.03) (end 99.90293 113.03) (width 1) (layer B.Cu) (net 9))
 (segment (start 91.44 118.92) (end 97.33 113.03) (width 1) (layer B.Cu) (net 9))
 (segment (start 91.44 121.92) (end 91.44 118.92) (width 1) (layer B.Cu) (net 9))
 (segment (start 65.84 104.34) (end 66.04 104.14) (width 1) (layer B.Cu) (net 11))
 (segment (start 61.16 99.51) (end 61.16 104.34) (width 1) (layer B.Cu) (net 11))
 (segment (start 80.83 79.84) (end 61.16 99.51) (width 1) (layer B.Cu) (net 11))
 (segment (start 80.83 77.84) (end 80.83 79.84) (width 1) (layer B.Cu) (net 11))
 (segment (start 56.29 104.34) (end 61.16 104.34) (width 1) (layer B.Cu) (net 11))
 (segment (start 61.16 104.34) (end 65.84 104.34) (width 1) (layer B.Cu) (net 11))
 (segment (start 56.29 77.88) (end 56.33 77.84) (width 1) (layer B.Cu) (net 13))
 (segment (start 56.29 89.18) (end 56.29 77.88) (width 1) (layer B.Cu) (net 13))
 (segment (start 56.29 99.18) (end 56.29 94.18) (width 1) (layer B.Cu) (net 14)))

